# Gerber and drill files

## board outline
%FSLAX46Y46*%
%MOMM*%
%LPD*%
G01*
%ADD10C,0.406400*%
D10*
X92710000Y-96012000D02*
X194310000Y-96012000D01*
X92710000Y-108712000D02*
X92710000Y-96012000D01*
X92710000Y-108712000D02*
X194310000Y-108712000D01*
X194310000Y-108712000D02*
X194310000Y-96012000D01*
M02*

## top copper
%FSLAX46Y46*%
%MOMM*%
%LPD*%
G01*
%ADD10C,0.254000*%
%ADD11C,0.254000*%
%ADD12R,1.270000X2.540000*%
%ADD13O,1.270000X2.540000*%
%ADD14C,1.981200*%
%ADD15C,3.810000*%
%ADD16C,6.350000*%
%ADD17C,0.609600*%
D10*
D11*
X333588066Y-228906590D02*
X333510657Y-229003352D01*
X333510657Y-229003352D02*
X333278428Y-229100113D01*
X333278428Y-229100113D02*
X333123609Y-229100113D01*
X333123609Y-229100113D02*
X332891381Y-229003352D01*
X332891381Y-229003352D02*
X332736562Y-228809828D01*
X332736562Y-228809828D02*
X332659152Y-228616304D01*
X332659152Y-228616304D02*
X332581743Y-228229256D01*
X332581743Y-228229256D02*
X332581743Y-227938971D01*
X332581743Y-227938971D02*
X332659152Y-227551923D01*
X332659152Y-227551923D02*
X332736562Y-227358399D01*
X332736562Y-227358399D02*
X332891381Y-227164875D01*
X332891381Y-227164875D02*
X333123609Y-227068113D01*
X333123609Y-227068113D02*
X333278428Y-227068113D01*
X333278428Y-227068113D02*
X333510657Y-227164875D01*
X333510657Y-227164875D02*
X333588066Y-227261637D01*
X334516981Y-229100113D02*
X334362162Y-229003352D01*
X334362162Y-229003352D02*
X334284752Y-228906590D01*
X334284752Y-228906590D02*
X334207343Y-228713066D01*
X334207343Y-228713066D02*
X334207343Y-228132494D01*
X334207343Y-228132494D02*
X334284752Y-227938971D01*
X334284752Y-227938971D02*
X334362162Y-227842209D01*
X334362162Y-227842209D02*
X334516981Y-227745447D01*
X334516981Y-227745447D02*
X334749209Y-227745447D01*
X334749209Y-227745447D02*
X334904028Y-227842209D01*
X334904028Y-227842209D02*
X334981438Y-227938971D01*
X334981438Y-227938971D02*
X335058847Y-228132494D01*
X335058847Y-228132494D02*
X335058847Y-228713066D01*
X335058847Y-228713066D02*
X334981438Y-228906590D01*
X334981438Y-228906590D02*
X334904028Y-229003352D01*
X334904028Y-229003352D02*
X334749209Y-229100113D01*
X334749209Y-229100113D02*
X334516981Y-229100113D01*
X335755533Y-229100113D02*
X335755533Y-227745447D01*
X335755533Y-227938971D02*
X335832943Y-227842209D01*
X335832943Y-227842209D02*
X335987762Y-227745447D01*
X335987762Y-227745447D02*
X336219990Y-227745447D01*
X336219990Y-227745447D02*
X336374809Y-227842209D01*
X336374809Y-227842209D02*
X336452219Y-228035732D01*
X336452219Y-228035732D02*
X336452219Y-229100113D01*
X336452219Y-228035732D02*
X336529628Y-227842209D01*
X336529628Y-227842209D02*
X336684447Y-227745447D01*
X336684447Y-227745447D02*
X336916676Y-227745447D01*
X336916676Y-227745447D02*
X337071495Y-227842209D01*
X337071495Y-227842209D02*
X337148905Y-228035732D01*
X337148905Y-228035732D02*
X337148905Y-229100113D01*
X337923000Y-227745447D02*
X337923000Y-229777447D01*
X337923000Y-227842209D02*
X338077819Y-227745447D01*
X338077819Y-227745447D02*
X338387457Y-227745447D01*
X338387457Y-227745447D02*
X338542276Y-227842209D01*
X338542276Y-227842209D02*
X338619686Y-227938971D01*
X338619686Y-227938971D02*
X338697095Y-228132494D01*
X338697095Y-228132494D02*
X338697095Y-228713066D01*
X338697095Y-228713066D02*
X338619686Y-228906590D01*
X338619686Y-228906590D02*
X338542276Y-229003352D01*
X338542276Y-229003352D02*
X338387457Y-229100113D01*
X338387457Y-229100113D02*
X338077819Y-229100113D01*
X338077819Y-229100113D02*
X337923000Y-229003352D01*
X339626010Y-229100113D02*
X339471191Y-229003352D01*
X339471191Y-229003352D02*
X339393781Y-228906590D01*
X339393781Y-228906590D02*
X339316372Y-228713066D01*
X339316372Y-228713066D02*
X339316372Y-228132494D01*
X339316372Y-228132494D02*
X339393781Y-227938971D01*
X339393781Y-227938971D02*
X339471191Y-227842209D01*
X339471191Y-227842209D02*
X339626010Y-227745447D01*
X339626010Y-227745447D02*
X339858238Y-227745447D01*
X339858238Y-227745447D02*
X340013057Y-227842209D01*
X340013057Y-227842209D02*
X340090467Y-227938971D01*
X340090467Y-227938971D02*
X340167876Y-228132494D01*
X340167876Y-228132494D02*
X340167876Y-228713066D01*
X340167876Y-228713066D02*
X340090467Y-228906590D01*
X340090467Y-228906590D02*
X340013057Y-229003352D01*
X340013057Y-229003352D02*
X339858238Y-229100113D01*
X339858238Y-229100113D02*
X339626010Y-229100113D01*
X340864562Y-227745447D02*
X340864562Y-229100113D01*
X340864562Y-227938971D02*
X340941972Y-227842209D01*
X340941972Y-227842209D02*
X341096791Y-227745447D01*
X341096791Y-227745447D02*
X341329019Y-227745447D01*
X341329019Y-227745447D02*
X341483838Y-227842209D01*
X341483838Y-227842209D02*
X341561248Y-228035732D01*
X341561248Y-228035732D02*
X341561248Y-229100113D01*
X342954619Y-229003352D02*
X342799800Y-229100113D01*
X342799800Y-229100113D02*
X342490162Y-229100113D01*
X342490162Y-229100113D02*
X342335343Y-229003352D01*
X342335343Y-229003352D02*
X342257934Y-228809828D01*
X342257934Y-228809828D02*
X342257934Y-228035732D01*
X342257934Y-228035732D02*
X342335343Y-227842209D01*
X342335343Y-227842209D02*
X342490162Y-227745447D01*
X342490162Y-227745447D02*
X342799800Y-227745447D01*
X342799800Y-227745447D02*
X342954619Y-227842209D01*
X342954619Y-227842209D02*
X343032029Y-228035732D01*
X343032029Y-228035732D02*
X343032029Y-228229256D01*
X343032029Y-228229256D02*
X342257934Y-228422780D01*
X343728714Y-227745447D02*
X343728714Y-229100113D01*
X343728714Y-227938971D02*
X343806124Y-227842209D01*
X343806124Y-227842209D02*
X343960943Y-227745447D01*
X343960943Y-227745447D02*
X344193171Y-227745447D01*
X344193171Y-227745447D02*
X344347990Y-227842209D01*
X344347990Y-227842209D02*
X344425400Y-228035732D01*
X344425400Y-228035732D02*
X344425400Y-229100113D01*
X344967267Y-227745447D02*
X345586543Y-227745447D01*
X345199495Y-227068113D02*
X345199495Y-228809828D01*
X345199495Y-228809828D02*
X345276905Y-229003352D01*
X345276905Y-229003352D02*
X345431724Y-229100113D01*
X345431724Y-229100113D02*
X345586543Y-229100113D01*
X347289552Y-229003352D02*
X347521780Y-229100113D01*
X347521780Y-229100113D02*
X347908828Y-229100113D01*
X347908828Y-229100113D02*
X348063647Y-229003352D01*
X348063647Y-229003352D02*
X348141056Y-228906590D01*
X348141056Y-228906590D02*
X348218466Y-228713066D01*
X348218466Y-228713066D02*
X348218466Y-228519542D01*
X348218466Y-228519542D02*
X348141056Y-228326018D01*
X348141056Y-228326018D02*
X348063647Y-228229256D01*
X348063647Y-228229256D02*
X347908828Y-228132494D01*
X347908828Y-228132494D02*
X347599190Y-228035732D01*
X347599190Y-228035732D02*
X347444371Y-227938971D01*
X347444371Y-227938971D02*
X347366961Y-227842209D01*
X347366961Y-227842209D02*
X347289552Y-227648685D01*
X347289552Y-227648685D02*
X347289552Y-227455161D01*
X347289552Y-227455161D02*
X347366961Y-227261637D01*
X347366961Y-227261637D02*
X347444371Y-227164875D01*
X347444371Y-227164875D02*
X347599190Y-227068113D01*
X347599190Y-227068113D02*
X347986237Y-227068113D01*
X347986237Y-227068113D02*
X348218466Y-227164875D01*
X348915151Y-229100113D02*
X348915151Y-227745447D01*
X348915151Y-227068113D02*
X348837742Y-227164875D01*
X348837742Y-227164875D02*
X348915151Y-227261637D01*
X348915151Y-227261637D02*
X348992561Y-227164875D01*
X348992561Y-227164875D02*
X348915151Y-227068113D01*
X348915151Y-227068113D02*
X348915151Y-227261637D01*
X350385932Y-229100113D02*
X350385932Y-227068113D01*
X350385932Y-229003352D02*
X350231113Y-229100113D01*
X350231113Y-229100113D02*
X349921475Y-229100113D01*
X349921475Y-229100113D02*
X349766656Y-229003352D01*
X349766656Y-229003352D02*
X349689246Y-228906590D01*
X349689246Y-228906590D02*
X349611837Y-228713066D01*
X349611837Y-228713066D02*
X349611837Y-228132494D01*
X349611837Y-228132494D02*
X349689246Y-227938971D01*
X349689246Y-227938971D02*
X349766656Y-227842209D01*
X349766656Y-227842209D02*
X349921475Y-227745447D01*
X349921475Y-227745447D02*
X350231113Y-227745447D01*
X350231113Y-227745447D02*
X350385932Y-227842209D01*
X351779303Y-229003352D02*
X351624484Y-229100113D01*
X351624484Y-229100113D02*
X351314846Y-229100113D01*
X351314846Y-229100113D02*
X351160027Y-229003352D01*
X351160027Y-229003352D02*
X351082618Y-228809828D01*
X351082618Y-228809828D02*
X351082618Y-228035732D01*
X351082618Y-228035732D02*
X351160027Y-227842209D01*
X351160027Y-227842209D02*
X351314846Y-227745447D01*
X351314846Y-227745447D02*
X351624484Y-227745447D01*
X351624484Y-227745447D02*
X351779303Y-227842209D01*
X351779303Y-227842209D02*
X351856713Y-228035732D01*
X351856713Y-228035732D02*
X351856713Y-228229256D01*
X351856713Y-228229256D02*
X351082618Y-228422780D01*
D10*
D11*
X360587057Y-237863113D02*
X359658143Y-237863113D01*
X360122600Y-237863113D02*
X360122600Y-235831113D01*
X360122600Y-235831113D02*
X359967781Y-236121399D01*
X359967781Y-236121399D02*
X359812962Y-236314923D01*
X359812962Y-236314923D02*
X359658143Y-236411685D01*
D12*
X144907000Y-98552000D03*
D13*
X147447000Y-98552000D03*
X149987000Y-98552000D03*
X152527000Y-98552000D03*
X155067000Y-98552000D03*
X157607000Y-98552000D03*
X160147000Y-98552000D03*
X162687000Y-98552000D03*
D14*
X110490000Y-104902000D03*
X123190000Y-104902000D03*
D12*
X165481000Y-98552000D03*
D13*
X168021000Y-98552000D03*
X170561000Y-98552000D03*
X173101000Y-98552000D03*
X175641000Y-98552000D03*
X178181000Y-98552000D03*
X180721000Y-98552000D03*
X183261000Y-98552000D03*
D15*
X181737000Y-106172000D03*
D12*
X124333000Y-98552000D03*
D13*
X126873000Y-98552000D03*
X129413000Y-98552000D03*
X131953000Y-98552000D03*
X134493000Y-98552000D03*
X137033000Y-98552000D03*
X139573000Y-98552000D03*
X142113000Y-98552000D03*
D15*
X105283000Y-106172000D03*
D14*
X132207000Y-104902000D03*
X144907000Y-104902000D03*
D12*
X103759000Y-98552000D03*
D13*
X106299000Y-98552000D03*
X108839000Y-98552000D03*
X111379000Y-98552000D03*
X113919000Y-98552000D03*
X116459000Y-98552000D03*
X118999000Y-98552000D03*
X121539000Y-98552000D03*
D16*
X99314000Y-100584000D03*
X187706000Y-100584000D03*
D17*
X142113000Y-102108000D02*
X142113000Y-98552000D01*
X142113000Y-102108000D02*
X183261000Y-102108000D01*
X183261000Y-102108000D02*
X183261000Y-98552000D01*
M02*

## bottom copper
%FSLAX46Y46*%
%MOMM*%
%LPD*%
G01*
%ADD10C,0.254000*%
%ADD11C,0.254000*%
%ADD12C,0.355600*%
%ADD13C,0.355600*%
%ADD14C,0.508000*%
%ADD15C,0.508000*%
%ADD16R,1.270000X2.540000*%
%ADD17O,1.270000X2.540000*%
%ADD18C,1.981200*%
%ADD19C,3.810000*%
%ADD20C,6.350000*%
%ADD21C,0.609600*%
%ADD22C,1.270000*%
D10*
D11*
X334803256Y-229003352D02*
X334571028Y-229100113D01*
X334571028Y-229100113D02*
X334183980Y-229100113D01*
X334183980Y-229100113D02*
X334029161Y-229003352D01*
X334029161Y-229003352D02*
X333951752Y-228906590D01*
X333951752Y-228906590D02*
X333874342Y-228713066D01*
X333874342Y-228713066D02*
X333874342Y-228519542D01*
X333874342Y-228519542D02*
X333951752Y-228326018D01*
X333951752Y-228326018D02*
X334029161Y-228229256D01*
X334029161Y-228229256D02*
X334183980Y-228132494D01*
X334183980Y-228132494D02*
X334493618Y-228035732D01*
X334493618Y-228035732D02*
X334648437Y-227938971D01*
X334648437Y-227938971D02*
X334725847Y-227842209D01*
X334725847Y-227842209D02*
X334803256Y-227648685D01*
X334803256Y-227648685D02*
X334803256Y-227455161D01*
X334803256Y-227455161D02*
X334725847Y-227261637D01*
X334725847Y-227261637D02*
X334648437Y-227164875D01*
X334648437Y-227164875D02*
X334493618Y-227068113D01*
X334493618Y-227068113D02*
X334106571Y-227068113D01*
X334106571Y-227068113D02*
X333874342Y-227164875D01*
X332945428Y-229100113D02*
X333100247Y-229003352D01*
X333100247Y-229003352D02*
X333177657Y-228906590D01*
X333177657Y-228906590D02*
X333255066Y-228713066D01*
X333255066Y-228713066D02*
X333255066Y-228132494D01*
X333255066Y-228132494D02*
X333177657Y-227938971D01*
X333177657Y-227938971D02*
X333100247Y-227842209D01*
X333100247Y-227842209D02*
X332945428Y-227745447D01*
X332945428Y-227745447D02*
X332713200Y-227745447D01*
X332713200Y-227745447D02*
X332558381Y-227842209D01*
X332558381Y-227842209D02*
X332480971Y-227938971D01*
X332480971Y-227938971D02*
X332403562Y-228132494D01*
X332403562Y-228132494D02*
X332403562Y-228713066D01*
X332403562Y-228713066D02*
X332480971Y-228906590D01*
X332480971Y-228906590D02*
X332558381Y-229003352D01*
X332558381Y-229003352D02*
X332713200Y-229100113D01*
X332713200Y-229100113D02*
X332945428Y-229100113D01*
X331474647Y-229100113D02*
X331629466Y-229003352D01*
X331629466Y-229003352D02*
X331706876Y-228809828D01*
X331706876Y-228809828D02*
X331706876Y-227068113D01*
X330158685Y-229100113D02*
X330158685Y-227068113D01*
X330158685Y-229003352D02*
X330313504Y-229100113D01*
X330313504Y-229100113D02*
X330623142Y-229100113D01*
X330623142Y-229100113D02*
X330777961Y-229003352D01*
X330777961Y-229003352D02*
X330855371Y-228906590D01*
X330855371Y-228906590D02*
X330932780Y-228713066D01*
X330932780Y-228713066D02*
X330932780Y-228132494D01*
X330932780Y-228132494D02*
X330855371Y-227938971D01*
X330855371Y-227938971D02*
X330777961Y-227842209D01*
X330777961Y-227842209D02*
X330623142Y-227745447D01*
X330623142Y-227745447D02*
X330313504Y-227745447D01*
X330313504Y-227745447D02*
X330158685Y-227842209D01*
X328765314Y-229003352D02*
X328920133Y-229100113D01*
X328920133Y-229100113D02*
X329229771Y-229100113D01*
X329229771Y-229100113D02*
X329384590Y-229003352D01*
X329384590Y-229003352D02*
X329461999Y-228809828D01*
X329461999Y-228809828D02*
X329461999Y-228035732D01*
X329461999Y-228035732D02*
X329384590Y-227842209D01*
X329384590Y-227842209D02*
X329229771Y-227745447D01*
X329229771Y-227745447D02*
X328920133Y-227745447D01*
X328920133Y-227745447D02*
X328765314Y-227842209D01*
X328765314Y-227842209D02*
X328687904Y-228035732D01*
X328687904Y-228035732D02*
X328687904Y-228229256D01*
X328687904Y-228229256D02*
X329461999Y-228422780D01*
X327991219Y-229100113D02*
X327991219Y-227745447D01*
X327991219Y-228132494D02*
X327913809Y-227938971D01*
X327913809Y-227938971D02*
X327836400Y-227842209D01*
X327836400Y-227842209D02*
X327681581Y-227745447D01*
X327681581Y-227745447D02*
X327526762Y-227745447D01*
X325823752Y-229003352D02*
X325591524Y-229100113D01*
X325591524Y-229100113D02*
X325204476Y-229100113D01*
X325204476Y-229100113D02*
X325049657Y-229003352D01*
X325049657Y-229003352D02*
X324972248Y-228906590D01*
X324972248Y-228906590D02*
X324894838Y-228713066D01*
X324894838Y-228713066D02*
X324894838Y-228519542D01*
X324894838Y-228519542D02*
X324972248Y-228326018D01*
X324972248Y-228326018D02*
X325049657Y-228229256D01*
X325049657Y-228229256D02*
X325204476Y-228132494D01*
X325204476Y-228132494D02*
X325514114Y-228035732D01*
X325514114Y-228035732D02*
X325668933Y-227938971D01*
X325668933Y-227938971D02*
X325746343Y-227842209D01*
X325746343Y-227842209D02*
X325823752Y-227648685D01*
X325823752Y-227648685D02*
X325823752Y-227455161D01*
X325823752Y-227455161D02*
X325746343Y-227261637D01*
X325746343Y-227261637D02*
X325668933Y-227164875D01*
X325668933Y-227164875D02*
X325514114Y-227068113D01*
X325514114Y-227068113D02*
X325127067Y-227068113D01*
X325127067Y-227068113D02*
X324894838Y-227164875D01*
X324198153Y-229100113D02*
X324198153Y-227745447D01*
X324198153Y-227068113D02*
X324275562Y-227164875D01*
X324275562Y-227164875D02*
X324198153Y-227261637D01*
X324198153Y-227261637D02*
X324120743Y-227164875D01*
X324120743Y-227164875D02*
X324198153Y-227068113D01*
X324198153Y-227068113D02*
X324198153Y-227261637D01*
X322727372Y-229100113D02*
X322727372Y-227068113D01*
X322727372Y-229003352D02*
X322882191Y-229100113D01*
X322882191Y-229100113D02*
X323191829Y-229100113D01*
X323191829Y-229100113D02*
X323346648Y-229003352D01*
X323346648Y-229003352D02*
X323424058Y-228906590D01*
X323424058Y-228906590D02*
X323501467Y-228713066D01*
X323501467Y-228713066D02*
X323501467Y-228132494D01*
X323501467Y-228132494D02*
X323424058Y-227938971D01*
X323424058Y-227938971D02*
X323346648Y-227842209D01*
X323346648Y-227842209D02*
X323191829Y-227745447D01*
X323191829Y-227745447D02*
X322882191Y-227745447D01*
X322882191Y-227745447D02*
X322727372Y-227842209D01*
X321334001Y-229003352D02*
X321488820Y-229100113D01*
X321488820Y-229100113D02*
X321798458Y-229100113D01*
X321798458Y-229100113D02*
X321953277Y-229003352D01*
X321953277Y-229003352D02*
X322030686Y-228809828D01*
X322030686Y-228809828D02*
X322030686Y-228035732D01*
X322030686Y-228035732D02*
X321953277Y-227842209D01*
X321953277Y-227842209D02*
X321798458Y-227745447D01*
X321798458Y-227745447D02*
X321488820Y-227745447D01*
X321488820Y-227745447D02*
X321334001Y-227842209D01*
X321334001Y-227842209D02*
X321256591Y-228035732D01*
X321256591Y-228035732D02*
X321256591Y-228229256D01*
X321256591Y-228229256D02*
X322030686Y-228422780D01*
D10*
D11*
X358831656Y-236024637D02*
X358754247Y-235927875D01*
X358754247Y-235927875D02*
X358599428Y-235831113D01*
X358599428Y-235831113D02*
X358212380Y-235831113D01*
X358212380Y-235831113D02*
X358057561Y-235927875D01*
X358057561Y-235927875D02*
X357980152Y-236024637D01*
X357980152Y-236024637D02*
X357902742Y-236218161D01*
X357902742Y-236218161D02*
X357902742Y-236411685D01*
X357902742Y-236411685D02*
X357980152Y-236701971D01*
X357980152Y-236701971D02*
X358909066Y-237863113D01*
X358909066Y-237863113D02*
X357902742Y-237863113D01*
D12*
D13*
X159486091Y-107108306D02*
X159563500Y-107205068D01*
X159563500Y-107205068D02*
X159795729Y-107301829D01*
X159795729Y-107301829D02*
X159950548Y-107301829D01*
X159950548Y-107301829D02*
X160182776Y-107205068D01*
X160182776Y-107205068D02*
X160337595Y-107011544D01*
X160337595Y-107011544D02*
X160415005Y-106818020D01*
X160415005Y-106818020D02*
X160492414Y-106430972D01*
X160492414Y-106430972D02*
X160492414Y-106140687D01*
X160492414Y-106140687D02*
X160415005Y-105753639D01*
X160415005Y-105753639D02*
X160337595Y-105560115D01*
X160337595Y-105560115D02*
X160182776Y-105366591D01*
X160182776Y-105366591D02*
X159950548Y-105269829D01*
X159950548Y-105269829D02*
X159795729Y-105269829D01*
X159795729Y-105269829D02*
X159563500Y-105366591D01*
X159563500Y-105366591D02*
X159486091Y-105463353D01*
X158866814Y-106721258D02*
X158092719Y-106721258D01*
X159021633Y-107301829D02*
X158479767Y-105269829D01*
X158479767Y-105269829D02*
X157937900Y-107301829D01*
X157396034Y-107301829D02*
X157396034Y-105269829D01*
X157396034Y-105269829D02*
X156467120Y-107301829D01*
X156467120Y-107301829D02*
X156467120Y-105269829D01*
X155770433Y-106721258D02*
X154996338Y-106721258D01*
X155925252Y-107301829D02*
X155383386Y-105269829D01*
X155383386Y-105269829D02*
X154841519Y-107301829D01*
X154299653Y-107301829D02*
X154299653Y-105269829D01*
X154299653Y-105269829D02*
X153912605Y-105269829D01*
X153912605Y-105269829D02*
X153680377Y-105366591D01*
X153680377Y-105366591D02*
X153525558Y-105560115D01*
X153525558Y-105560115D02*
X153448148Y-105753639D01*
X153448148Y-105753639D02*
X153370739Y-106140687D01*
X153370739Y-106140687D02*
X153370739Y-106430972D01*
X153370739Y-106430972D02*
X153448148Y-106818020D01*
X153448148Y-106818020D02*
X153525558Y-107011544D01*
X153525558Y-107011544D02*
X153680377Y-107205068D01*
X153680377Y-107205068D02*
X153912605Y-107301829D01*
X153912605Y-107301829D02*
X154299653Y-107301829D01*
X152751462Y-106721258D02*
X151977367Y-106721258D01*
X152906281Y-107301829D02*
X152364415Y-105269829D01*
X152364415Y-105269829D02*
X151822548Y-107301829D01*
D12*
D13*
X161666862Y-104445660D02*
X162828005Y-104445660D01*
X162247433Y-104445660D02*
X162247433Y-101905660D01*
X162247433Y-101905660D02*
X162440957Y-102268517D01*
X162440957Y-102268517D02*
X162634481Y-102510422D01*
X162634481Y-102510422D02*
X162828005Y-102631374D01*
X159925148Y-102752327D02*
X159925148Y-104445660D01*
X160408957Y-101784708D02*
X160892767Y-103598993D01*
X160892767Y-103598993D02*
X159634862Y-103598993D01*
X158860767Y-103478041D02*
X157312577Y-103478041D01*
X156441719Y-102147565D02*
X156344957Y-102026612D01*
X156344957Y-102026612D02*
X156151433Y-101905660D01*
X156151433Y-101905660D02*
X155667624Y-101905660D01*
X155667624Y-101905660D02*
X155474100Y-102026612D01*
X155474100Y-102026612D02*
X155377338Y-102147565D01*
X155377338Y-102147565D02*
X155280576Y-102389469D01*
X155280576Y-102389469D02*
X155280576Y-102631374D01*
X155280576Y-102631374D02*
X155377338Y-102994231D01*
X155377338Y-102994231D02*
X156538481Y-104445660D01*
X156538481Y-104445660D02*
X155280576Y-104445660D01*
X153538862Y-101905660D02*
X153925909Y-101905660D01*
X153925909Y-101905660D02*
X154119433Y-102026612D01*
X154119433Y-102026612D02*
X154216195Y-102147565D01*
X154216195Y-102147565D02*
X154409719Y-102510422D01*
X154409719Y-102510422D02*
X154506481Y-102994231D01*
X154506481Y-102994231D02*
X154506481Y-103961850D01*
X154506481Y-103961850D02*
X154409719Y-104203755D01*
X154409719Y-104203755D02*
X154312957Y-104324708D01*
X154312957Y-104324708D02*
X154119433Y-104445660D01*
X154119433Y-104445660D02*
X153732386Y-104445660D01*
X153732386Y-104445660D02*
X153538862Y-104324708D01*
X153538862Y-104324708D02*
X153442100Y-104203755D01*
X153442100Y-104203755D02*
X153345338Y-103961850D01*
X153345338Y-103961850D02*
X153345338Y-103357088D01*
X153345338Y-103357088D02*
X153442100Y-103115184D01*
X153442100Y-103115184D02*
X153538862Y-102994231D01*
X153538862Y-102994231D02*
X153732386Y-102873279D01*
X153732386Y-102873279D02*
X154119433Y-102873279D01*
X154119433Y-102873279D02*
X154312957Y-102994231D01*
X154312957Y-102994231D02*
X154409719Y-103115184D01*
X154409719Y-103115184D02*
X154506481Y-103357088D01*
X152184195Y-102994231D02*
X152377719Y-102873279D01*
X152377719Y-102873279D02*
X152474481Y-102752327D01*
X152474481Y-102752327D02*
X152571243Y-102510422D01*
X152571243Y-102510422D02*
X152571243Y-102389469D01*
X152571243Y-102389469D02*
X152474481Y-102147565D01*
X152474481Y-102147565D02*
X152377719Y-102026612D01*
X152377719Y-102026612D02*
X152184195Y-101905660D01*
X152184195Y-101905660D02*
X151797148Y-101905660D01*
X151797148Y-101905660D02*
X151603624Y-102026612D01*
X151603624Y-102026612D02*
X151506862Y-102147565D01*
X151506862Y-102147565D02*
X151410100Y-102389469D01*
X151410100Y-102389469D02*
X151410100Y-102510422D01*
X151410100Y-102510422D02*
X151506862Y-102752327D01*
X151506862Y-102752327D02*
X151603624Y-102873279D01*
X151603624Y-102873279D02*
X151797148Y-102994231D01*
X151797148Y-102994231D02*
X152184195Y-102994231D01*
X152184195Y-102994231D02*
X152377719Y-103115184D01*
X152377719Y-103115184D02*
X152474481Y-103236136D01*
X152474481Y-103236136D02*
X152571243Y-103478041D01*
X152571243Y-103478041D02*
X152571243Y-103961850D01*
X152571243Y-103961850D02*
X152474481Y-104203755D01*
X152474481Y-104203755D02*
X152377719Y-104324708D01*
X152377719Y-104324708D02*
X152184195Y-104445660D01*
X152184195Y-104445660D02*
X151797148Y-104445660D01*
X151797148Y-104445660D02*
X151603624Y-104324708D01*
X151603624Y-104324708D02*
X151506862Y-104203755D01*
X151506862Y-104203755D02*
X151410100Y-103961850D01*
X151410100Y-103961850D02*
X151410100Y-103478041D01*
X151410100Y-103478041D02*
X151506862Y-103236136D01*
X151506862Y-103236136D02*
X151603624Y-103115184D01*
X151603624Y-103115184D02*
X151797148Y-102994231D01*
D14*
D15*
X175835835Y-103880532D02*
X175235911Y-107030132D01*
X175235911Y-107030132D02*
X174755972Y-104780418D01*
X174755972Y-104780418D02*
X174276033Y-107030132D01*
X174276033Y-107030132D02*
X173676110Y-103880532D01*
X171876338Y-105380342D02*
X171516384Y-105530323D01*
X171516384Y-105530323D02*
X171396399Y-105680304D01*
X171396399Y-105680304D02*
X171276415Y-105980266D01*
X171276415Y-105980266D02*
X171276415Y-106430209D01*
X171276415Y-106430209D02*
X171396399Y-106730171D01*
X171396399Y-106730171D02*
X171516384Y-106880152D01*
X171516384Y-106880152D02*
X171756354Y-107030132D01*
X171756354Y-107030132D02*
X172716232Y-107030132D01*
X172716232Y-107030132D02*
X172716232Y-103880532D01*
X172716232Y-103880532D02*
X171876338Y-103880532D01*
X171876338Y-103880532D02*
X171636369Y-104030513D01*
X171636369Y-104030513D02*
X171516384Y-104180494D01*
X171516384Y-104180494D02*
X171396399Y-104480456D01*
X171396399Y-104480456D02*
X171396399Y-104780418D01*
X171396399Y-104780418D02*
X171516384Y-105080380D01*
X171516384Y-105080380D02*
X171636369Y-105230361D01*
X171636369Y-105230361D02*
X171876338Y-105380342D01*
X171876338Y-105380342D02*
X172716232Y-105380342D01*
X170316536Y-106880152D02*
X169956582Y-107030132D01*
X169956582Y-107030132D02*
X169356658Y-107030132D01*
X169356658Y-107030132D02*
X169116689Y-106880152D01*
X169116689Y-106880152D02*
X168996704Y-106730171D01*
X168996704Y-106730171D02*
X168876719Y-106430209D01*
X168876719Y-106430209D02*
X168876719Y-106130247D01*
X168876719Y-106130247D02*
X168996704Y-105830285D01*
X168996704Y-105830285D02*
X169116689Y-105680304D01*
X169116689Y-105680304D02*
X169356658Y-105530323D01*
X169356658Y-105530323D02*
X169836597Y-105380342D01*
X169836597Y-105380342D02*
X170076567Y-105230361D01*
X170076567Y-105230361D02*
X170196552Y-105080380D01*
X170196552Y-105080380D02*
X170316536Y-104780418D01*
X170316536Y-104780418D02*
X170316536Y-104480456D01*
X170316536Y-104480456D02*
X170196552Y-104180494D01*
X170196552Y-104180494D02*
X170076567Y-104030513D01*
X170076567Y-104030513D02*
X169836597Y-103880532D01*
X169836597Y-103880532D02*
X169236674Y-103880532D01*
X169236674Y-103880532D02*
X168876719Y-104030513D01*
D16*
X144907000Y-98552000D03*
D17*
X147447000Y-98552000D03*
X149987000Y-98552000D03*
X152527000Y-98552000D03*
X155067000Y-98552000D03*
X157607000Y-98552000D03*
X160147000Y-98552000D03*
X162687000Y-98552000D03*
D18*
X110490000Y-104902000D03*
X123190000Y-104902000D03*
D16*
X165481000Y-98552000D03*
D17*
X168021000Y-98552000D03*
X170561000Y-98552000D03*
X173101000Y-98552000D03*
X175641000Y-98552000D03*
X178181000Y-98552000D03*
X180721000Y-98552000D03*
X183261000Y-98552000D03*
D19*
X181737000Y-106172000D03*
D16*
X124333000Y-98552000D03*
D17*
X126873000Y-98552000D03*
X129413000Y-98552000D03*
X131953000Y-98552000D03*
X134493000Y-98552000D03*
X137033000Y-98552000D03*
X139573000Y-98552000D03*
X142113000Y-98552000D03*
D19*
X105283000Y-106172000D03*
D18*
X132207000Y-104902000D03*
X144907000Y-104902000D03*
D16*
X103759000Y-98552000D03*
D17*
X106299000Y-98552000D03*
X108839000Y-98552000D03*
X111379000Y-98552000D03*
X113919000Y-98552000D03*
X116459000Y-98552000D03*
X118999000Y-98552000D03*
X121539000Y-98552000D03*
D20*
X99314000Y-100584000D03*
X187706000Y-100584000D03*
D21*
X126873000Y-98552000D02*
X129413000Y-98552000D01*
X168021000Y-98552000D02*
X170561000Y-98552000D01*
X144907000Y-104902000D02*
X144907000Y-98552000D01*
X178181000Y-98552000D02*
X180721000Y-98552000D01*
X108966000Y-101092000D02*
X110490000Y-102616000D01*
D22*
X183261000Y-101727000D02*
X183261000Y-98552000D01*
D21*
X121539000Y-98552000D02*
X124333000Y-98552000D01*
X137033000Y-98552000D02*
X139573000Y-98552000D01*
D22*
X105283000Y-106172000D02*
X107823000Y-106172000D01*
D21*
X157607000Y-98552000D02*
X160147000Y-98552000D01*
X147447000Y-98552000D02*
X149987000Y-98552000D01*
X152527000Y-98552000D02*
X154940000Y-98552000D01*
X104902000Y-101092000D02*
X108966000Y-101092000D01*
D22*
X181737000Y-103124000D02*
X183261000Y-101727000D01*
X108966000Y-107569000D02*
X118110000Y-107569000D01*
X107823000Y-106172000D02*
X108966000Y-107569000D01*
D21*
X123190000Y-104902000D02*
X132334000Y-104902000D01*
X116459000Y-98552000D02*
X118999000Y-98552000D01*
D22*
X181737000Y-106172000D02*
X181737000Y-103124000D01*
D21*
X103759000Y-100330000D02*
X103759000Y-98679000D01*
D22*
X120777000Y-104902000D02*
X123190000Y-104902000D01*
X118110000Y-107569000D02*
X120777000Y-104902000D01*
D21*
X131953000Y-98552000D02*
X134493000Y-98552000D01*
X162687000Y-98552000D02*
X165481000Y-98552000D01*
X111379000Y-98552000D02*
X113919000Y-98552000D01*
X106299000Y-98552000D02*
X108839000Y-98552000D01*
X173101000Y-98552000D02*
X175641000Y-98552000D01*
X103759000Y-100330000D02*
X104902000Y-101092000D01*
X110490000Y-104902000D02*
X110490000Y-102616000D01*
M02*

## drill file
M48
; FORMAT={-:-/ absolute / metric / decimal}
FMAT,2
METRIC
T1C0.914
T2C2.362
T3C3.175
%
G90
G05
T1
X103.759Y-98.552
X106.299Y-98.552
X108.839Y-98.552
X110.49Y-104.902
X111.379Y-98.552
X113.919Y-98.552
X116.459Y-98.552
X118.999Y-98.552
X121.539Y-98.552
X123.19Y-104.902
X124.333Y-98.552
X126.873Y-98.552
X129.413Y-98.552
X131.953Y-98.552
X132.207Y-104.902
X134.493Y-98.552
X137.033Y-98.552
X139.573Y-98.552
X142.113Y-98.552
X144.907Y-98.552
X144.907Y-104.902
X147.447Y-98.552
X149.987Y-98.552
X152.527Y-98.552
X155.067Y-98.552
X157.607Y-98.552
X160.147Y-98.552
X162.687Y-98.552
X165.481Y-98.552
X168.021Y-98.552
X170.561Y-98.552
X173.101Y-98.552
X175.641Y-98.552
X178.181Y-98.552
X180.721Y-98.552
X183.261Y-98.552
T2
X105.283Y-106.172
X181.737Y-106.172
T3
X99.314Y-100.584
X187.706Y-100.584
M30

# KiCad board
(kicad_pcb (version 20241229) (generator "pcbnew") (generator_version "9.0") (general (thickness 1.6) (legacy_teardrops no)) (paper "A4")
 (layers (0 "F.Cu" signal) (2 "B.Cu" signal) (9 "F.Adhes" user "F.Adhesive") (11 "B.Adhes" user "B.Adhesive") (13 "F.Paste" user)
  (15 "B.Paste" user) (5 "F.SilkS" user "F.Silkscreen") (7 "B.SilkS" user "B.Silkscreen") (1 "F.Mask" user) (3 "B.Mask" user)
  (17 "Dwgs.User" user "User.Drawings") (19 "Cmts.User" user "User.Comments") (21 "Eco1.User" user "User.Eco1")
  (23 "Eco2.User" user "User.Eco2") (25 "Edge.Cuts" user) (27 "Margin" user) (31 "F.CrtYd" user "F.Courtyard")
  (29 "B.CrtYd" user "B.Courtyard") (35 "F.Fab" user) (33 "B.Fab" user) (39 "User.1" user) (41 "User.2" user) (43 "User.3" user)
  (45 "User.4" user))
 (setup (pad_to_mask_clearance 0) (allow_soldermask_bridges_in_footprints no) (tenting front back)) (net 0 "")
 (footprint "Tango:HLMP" (layer "F.Cu") (at 144.907 98.679)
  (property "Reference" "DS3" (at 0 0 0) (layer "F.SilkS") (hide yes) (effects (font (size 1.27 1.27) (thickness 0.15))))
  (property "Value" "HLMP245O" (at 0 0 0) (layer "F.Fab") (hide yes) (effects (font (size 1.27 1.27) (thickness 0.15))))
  (pad "1" thru_hole rect (at 0 -0.127) (size 1.27 2.54) (drill 0.9144) (layers "*.Cu" "*.Mask") (remove_unused_layers no)
   (thermal_bridge_angle 45))
  (pad "2" thru_hole oval (at 2.54 -0.127) (size 1.27 2.54) (drill 0.9144) (layers "*.Cu" "*.Mask") (remove_unused_layers no)
   (thermal_bridge_angle 45))
  (pad "3" thru_hole oval (at 5.08 -0.127) (size 1.27 2.54) (drill 0.9144) (layers "*.Cu" "*.Mask") (remove_unused_layers no)
   (thermal_bridge_angle 45))
  (pad "4" thru_hole oval (at 7.62 -0.127) (size 1.27 2.54) (drill 0.9144) (layers "*.Cu" "*.Mask") (remove_unused_layers no)
   (thermal_bridge_angle 45))
  (pad "5" thru_hole oval (at 10.16 -0.127) (size 1.27 2.54) (drill 0.9144) (layers "*.Cu" "*.Mask") (remove_unused_layers no)
   (thermal_bridge_angle 45))
  (pad "6" thru_hole oval (at 12.7 -0.127) (size 1.27 2.54) (drill 0.9144) (layers "*.Cu" "*.Mask") (remove_unused_layers no)
   (thermal_bridge_angle 45))
  (pad "7" thru_hole oval (at 15.24 -0.127) (size 1.27 2.54) (drill 0.9144) (layers "*.Cu" "*.Mask") (remove_unused_layers no)
   (thermal_bridge_angle 45))
  (pad "8" thru_hole oval (at 17.78 -0.127) (size 1.27 2.54) (drill 0.9144) (layers "*.Cu" "*.Mask") (remove_unused_layers no)
   (thermal_bridge_angle 45)))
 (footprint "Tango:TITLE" (layer "F.Cu") (at 381 238.887)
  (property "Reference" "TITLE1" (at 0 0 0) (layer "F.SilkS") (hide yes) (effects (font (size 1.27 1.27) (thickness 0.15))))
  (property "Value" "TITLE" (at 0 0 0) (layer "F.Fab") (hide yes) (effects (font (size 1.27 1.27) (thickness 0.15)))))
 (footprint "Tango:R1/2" (layer "F.Cu") (at 110.49 104.902)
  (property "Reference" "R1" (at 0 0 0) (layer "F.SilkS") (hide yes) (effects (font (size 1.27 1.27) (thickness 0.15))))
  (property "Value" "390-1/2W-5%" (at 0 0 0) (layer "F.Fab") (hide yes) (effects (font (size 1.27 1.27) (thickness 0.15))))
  (pad "1" thru_hole circle (at 0 0) (size 1.9812 1.9812) (drill 0.9144) (layers "*.Cu" "*.Mask") (remove_unused_layers no))
  (pad "2" thru_hole circle (at 12.7 0) (size 1.9812 1.9812) (drill 0.9144) (layers "*.Cu" "*.Mask") (remove_unused_layers no)))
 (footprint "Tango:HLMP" (layer "F.Cu") (at 165.481 98.679)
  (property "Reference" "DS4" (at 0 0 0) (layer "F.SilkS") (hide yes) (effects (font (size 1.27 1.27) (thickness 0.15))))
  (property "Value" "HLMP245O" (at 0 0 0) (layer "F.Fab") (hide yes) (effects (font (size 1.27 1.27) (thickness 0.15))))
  (pad "1" thru_hole rect (at 0 -0.127) (size 1.27 2.54) (drill 0.9144) (layers "*.Cu" "*.Mask") (remove_unused_layers no)
   (thermal_bridge_angle 45))
  (pad "2" thru_hole oval (at 2.54 -0.127) (size 1.27 2.54) (drill 0.9144) (layers "*.Cu" "*.Mask") (remove_unused_layers no)
   (thermal_bridge_angle 45))
  (pad "3" thru_hole oval (at 5.08 -0.127) (size 1.27 2.54) (drill 0.9144) (layers "*.Cu" "*.Mask") (remove_unused_layers no)
   (thermal_bridge_angle 45))
  (pad "4" thru_hole oval (at 7.62 -0.127) (size 1.27 2.54) (drill 0.9144) (layers "*.Cu" "*.Mask") (remove_unused_layers no)
   (thermal_bridge_angle 45))
  (pad "5" thru_hole oval (at 10.16 -0.127) (size 1.27 2.54) (drill 0.9144) (layers "*.Cu" "*.Mask") (remove_unused_layers no)
   (thermal_bridge_angle 45))
  (pad "6" thru_hole oval (at 12.7 -0.127) (size 1.27 2.54) (drill 0.9144) (layers "*.Cu" "*.Mask") (remove_unused_layers no)
   (thermal_bridge_angle 45))
  (pad "7" thru_hole oval (at 15.24 -0.127) (size 1.27 2.54) (drill 0.9144) (layers "*.Cu" "*.Mask") (remove_unused_layers no)
   (thermal_bridge_angle 45))
  (pad "8" thru_hole oval (at 17.78 -0.127) (size 1.27 2.54) (drill 0.9144) (layers "*.Cu" "*.Mask") (remove_unused_layers no)
   (thermal_bridge_angle 45)))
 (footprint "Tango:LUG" (layer "F.Cu") (at 181.737 106.172)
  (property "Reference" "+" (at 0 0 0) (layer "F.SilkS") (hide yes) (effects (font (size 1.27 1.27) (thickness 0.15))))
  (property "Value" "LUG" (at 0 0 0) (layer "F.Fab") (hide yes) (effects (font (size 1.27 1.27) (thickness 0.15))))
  (pad "1" thru_hole circle (at 0 0) (size 3.81 3.81) (drill 2.3622) (layers "*.Cu" "*.Mask") (remove_unused_layers no)))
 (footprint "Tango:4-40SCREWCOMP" (layer "F.Cu") (at 99.314 100.584)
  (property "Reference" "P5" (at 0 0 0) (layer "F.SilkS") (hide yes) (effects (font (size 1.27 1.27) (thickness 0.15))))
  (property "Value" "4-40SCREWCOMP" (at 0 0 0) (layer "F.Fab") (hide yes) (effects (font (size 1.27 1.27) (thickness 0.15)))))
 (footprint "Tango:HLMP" (layer "F.Cu") (at 124.333 98.679)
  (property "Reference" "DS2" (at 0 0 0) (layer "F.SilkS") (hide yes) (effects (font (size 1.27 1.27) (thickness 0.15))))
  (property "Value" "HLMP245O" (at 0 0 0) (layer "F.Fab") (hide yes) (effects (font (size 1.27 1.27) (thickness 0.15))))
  (pad "1" thru_hole rect (at 0 -0.127) (size 1.27 2.54) (drill 0.9144) (layers "*.Cu" "*.Mask") (remove_unused_layers no)
   (thermal_bridge_angle 45))
  (pad "2" thru_hole oval (at 2.54 -0.127) (size 1.27 2.54) (drill 0.9144) (layers "*.Cu" "*.Mask") (remove_unused_layers no)
   (thermal_bridge_angle 45))
  (pad "3" thru_hole oval (at 5.08 -0.127) (size 1.27 2.54) (drill 0.9144) (layers "*.Cu" "*.Mask") (remove_unused_layers no)
   (thermal_bridge_angle 45))
  (pad "4" thru_hole oval (at 7.62 -0.127) (size 1.27 2.54) (drill 0.9144) (layers "*.Cu" "*.Mask") (remove_unused_layers no)
   (thermal_bridge_angle 45))
  (pad "5" thru_hole oval (at 10.16 -0.127) (size 1.27 2.54) (drill 0.9144) (layers "*.Cu" "*.Mask") (remove_unused_layers no)
   (thermal_bridge_angle 45))
  (pad "6" thru_hole oval (at 12.7 -0.127) (size 1.27 2.54) (drill 0.9144) (layers "*.Cu" "*.Mask") (remove_unused_layers no)
   (thermal_bridge_angle 45))
  (pad "7" thru_hole oval (at 15.24 -0.127) (size 1.27 2.54) (drill 0.9144) (layers "*.Cu" "*.Mask") (remove_unused_layers no)
   (thermal_bridge_angle 45))
  (pad "8" thru_hole oval (at 17.78 -0.127) (size 1.27 2.54) (drill 0.9144) (layers "*.Cu" "*.Mask") (remove_unused_layers no)
   (thermal_bridge_angle 45)))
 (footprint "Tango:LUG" (layer "F.Cu") (at 105.283 106.172)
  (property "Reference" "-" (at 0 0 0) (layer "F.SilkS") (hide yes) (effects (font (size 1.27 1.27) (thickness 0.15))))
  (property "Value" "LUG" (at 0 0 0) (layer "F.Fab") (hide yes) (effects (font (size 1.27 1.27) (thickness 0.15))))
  (pad "1" thru_hole circle (at 0 0) (size 3.81 3.81) (drill 2.3622) (layers "*.Cu" "*.Mask") (remove_unused_layers no)))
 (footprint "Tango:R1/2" (layer "F.Cu") (at 132.207 104.902)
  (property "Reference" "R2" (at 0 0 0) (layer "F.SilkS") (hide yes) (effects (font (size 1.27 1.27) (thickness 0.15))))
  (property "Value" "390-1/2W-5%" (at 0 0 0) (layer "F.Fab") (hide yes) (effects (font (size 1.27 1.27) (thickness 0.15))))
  (pad "1" thru_hole circle (at 0 0) (size 1.9812 1.9812) (drill 0.9144) (layers "*.Cu" "*.Mask") (remove_unused_layers no))
  (pad "2" thru_hole circle (at 12.7 0) (size 1.9812 1.9812) (drill 0.9144) (layers "*.Cu" "*.Mask") (remove_unused_layers no)))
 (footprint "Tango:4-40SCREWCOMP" (layer "F.Cu") (at 187.706 100.584)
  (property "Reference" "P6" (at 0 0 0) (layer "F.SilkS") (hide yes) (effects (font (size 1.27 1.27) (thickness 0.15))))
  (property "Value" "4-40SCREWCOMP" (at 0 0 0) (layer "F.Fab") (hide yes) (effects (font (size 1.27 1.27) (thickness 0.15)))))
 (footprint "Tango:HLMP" (layer "F.Cu") (at 103.759 98.679)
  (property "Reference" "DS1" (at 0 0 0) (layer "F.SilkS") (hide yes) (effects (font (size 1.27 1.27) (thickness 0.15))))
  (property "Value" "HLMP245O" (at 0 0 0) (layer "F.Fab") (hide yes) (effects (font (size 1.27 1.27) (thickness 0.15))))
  (pad "1" thru_hole rect (at 0 -0.127) (size 1.27 2.54) (drill 0.9144) (layers "*.Cu" "*.Mask") (remove_unused_layers no)
   (thermal_bridge_angle 45))
  (pad "2" thru_hole oval (at 2.54 -0.127) (size 1.27 2.54) (drill 0.9144) (layers "*.Cu" "*.Mask") (remove_unused_layers no)
   (thermal_bridge_angle 45))
  (pad "3" thru_hole oval (at 5.08 -0.127) (size 1.27 2.54) (drill 0.9144) (layers "*.Cu" "*.Mask") (remove_unused_layers no)
   (thermal_bridge_angle 45))
  (pad "4" thru_hole oval (at 7.62 -0.127) (size 1.27 2.54) (drill 0.9144) (layers "*.Cu" "*.Mask") (remove_unused_layers no)
   (thermal_bridge_angle 45))
  (pad "5" thru_hole oval (at 10.16 -0.127) (size 1.27 2.54) (drill 0.9144) (layers "*.Cu" "*.Mask") (remove_unused_layers no)
   (thermal_bridge_angle 45))
  (pad "6" thru_hole oval (at 12.7 -0.127) (size 1.27 2.54) (drill 0.9144) (layers "*.Cu" "*.Mask") (remove_unused_layers no)
   (thermal_bridge_angle 45))
  (pad "7" thru_hole oval (at 15.24 -0.127) (size 1.27 2.54) (drill 0.9144) (layers "*.Cu" "*.Mask") (remove_unused_layers no)
   (thermal_bridge_angle 45))
  (pad "8" thru_hole oval (at 17.78 -0.127) (size 1.27 2.54) (drill 0.9144) (layers "*.Cu" "*.Mask") (remove_unused_layers no)
   (thermal_bridge_angle 45)))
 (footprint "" (layer "F.Cu") (at 99.314 100.584)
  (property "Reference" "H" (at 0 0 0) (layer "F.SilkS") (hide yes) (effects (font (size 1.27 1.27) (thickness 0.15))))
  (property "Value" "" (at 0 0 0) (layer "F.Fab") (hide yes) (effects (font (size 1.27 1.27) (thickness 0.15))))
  (pad "" np_thru_hole circle (at 0 0) (size 6.35 6.35) (drill 3.175) (layers "*.Cu" "*.Mask"))
  (pad "" np_thru_hole circle (at 88.392 0) (size 6.35 6.35) (drill 3.175) (layers "*.Cu" "*.Mask")))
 (gr_line (start 92.71 96.012) (end 194.31 96.012) (stroke (width 0.4064) (type default)) (layer "Edge.Cuts"))
 (gr_line (start 92.71 108.712) (end 92.71 96.012) (stroke (width 0.4064) (type default)) (layer "Edge.Cuts"))
 (gr_line (start 92.71 108.712) (end 194.31 108.712) (stroke (width 0.4064) (type default)) (layer "Edge.Cuts"))
 (gr_line (start 194.31 108.712) (end 194.31 96.012) (stroke (width 0.4064) (type default)) (layer "Edge.Cuts"))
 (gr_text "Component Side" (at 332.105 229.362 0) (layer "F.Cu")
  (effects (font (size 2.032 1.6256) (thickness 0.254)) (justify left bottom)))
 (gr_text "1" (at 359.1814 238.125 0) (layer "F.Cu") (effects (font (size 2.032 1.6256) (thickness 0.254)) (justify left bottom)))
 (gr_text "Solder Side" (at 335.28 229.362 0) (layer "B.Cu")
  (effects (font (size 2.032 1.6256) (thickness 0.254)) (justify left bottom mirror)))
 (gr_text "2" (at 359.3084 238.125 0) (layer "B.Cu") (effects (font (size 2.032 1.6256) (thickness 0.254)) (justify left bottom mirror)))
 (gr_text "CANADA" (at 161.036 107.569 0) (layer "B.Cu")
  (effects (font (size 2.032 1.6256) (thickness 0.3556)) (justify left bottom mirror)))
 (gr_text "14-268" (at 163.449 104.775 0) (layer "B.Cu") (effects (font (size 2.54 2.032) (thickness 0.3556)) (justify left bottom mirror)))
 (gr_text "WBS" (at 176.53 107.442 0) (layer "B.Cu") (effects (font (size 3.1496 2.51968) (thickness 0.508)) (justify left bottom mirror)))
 (segment (start 142.113 102.108) (end 142.113 98.552) (width 0.6096) (layer "F.Cu") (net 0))
 (segment (start 142.113 102.108) (end 183.261 102.108) (width 0.6096) (layer "F.Cu") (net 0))
 (segment (start 183.261 102.108) (end 183.261 98.552) (width 0.6096) (layer "F.Cu") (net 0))
 (segment (start 126.873 98.552) (end 129.413 98.552) (width 0.6096) (layer "B.Cu") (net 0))
 (segment (start 168.021 98.552) (end 170.561 98.552) (width 0.6096) (layer "B.Cu") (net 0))
 (segment (start 144.907 104.902) (end 144.907 98.552) (width 0.6096) (layer "B.Cu") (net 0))
 (segment (start 178.181 98.552) (end 180.721 98.552) (width 0.6096) (layer "B.Cu") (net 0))
 (segment (start 108.966 101.092) (end 110.49 102.616) (width 0.6096) (layer "B.Cu") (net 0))
 (segment (start 183.261 101.727) (end 183.261 98.552) (width 1.27) (layer "B.Cu") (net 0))
 (segment (start 121.539 98.552) (end 124.333 98.552) (width 0.6096) (layer "B.Cu") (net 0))
 (segment (start 137.033 98.552) (end 139.573 98.552) (width 0.6096) (layer "B.Cu") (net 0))
 (segment (start 105.283 106.172) (end 107.823 106.172) (width 1.27) (layer "B.Cu") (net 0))
 (segment (start 157.607 98.552) (end 160.147 98.552) (width 0.6096) (layer "B.Cu") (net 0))
 (segment (start 147.447 98.552) (end 149.987 98.552) (width 0.6096) (layer "B.Cu") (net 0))
 (segment (start 152.527 98.552) (end 154.94 98.552) (width 0.6096) (layer "B.Cu") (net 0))
 (segment (start 104.902 101.092) (end 108.966 101.092) (width 0.6096) (layer "B.Cu") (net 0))
 (segment (start 181.737 103.124) (end 183.261 101.727) (width 1.27) (layer "B.Cu") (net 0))
 (segment (start 108.966 107.569) (end 118.11 107.569) (width 1.27) (layer "B.Cu") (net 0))
 (segment (start 107.823 106.172) (end 108.966 107.569) (width 1.27) (layer "B.Cu") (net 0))
 (segment (start 123.19 104.902) (end 132.334 104.902) (width 0.6096) (layer "B.Cu") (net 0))
 (segment (start 116.459 98.552) (end 118.999 98.552) (width 0.6096) (layer "B.Cu") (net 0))
 (segment (start 181.737 106.172) (end 181.737 103.124) (width 1.27) (layer "B.Cu") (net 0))
 (segment (start 103.759 100.33) (end 103.759 98.679) (width 0.6096) (layer "B.Cu") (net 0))
 (segment (start 120.777 104.902) (end 123.19 104.902) (width 1.27) (layer "B.Cu") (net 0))
 (segment (start 118.11 107.569) (end 120.777 104.902) (width 1.27) (layer "B.Cu") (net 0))
 (segment (start 131.953 98.552) (end 134.493 98.552) (width 0.6096) (layer "B.Cu") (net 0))
 (segment (start 162.687 98.552) (end 165.481 98.552) (width 0.6096) (layer "B.Cu") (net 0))
 (segment (start 111.379 98.552) (end 113.919 98.552) (width 0.6096) (layer "B.Cu") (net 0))
 (segment (start 106.299 98.552) (end 108.839 98.552) (width 0.6096) (layer "B.Cu") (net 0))
 (segment (start 173.101 98.552) (end 175.641 98.552) (width 0.6096) (layer "B.Cu") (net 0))
 (segment (start 103.759 100.33) (end 104.902 101.092) (width 0.6096) (layer "B.Cu") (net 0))
 (segment (start 110.49 104.902) (end 110.49 102.616) (width 0.6096) (layer "B.Cu") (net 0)))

